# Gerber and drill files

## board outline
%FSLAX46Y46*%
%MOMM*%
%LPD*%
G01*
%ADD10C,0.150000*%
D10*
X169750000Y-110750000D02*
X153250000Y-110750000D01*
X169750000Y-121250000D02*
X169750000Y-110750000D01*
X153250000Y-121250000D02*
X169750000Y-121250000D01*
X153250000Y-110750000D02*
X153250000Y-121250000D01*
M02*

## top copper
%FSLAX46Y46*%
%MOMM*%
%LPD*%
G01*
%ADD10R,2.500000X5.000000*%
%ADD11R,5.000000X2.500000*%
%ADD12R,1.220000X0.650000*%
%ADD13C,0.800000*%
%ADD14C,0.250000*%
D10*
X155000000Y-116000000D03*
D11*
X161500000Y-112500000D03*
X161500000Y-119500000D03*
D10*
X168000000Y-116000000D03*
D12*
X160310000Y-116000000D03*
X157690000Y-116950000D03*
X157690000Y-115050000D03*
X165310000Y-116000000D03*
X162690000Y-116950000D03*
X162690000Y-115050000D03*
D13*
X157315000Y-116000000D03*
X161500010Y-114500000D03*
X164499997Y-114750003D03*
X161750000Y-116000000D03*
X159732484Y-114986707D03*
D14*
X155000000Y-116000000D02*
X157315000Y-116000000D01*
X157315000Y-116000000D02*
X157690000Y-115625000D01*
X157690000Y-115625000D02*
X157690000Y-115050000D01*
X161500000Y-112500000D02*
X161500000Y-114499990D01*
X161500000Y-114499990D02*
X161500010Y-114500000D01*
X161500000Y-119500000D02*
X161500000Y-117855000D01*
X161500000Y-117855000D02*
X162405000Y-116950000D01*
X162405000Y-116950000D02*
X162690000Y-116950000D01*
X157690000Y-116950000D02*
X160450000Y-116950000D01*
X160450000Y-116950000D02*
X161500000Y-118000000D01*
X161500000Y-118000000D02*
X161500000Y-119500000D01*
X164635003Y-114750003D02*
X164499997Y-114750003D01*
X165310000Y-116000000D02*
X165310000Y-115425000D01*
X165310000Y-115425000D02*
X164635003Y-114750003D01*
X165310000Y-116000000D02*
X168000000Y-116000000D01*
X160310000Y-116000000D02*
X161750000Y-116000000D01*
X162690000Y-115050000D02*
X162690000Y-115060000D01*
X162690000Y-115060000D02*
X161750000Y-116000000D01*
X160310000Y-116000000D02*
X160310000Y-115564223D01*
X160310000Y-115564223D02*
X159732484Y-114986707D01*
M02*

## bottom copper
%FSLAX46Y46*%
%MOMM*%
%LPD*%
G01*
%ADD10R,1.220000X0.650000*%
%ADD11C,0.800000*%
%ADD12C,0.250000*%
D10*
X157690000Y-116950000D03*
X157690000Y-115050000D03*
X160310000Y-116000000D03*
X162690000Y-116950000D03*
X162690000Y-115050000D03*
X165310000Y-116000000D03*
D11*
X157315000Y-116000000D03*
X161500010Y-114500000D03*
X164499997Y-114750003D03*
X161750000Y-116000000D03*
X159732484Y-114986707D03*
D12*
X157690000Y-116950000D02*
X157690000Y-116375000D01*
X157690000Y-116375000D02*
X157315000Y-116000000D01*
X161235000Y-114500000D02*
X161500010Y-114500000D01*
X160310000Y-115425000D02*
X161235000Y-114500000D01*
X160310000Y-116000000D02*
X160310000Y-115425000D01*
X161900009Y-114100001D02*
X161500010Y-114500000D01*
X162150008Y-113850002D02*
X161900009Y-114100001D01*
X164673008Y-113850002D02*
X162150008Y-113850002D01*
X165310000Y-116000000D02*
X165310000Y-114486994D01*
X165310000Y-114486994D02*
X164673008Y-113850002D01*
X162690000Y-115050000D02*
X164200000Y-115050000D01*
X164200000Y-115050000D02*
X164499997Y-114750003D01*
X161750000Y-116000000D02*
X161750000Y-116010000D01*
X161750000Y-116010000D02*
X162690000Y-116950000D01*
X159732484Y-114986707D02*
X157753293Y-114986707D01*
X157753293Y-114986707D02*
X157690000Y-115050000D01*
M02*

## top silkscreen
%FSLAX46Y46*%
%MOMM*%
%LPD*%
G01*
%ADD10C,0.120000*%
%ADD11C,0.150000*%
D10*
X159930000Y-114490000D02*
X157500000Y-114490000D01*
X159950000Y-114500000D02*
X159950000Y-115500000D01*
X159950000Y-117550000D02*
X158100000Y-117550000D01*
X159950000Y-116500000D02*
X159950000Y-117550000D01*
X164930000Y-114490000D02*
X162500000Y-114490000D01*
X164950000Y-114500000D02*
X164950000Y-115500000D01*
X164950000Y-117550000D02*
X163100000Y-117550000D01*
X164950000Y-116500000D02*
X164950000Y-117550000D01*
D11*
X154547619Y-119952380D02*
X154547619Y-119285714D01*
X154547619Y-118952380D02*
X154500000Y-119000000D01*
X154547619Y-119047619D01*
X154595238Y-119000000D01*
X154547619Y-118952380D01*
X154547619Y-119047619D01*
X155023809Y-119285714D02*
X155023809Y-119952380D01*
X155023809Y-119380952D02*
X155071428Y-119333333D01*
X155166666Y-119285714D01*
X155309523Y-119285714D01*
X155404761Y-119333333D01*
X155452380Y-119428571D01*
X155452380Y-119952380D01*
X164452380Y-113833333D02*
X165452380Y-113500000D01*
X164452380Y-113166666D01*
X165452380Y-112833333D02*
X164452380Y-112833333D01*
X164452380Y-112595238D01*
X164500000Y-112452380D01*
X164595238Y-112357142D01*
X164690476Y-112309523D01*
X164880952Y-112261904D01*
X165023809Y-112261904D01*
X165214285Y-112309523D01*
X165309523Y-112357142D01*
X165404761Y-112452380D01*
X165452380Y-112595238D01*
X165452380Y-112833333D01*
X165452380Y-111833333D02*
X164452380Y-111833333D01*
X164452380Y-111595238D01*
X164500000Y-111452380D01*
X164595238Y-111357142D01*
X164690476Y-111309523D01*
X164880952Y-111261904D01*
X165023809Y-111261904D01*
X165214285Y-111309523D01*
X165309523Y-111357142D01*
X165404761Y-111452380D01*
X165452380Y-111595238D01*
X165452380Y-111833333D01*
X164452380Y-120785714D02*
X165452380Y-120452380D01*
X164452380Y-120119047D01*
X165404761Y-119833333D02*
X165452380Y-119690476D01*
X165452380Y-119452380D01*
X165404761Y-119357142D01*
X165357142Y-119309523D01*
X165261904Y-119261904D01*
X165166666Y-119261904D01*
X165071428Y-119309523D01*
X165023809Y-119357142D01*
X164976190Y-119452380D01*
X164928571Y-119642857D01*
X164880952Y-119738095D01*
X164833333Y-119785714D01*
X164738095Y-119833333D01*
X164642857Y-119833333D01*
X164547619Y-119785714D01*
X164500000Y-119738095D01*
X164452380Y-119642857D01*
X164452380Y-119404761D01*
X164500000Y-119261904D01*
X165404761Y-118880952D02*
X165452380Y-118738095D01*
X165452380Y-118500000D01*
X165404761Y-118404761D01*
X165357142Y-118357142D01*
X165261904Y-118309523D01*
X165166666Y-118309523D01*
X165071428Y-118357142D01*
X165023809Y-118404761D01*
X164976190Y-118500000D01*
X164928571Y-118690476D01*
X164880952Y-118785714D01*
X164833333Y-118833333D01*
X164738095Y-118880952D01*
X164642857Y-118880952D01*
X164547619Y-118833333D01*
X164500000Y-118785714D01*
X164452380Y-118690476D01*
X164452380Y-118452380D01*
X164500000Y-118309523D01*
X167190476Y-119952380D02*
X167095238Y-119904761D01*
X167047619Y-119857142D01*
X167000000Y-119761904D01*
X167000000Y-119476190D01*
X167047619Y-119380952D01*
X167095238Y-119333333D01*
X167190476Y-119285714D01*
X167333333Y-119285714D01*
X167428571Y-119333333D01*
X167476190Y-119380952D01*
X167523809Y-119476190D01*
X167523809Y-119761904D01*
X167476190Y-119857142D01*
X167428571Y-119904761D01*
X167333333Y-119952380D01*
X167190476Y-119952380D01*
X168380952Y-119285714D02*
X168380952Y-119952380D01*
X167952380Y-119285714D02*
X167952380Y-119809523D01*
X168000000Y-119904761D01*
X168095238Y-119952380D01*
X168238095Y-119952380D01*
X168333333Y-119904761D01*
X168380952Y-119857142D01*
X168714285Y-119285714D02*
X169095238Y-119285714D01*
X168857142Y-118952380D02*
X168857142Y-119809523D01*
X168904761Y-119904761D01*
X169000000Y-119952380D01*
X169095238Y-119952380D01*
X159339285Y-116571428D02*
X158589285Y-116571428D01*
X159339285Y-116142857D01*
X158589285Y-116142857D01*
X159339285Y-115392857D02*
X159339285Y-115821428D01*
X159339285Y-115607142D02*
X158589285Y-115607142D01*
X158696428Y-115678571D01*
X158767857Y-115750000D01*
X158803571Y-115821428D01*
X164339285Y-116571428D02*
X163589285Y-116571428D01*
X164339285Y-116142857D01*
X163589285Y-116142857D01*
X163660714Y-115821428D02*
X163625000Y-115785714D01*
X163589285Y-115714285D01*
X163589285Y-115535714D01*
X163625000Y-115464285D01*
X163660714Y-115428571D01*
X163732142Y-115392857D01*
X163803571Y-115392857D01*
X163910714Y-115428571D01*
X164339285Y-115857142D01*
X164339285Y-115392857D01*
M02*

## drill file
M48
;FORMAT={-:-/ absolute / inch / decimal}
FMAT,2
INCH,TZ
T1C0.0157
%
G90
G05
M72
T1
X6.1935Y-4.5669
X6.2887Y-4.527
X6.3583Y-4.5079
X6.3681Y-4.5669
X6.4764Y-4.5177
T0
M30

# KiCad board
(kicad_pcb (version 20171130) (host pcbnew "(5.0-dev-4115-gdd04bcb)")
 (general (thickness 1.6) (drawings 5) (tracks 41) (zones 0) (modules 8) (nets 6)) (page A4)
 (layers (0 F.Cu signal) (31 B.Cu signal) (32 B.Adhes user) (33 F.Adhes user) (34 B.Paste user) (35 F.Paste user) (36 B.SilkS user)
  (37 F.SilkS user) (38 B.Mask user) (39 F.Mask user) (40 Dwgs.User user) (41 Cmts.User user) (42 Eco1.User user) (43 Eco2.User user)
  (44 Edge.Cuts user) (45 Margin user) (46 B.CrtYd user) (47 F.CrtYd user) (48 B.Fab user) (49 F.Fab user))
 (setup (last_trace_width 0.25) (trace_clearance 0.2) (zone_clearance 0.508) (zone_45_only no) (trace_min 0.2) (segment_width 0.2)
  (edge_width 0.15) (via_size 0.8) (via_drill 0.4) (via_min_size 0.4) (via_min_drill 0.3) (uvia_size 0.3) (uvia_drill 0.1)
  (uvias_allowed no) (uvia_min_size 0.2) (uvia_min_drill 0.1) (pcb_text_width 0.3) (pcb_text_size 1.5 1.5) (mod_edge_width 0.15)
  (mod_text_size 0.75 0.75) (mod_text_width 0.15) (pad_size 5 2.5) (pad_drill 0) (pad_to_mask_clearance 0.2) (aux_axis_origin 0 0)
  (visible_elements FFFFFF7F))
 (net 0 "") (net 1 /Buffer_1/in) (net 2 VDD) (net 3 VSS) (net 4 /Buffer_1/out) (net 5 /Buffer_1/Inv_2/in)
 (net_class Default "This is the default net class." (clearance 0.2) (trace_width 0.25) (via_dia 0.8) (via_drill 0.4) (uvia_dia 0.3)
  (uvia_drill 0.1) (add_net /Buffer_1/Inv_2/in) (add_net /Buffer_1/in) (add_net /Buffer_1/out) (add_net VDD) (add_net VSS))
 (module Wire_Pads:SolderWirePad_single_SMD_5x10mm (layer F.Cu) (at 155 116 90)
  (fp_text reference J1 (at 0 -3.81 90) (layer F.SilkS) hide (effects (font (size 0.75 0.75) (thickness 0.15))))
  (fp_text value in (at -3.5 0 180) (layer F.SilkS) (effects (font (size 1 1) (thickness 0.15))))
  (pad 1 smd rect (at 0 0 90) (size 5 2.5) (layers F.Cu F.Paste F.Mask) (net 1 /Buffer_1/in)))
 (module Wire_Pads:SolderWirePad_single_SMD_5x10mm (layer F.Cu) (at 161.5 112.5)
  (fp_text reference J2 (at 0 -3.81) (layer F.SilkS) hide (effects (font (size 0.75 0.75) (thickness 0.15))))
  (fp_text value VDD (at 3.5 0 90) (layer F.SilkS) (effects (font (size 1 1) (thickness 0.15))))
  (pad 1 smd rect (at 0 0) (size 5 2.5) (layers F.Cu F.Paste F.Mask) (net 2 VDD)))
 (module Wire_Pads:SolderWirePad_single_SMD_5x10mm (layer F.Cu) (at 161.5 119.5)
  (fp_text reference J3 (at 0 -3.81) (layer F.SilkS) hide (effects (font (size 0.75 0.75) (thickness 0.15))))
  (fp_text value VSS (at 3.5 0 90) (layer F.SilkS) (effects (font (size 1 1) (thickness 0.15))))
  (pad 1 smd rect (at 0 0) (size 5 2.5) (layers F.Cu F.Paste F.Mask) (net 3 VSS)))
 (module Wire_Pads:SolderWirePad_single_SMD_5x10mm (layer F.Cu) (at 168 116 90)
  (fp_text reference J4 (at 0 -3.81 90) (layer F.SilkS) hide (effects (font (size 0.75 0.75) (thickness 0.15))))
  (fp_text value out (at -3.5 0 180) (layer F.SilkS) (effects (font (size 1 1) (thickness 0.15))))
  (pad 1 smd rect (at 0 0 90) (size 5 2.5) (layers F.Cu F.Paste F.Mask) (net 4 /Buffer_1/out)))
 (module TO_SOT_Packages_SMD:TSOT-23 (layer F.Cu) (at 159 116)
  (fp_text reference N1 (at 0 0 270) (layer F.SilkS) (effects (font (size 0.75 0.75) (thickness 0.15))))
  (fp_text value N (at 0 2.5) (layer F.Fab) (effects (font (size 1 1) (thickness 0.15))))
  (fp_line (start 0.93 -1.51) (end -1.5 -1.51) (layer F.SilkS) (width 0.12))
  (fp_line (start 0.95 -1.5) (end 0.95 -0.5) (layer F.SilkS) (width 0.12))
  (fp_line (start 0.95 1.55) (end -0.9 1.55) (layer F.SilkS) (width 0.12))
  (fp_line (start 0.95 0.5) (end 0.95 1.55) (layer F.SilkS) (width 0.12))
  (pad 3 smd rect (at 1.31 0) (size 1.22 0.65) (layers F.Cu F.Paste F.Mask) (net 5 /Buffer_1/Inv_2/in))
  (pad 2 smd rect (at -1.31 0.95) (size 1.22 0.65) (layers F.Cu F.Paste F.Mask) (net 3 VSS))
  (pad 1 smd rect (at -1.31 -0.95) (size 1.22 0.65) (layers F.Cu F.Paste F.Mask) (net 1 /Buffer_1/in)))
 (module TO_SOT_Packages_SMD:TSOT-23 (layer F.Cu) (at 164 116)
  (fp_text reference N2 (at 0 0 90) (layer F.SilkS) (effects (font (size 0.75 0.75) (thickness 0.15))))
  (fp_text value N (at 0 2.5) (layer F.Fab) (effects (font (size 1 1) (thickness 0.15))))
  (fp_line (start 0.93 -1.51) (end -1.5 -1.51) (layer F.SilkS) (width 0.12))
  (fp_line (start 0.95 -1.5) (end 0.95 -0.5) (layer F.SilkS) (width 0.12))
  (fp_line (start 0.95 1.55) (end -0.9 1.55) (layer F.SilkS) (width 0.12))
  (fp_line (start 0.95 0.5) (end 0.95 1.55) (layer F.SilkS) (width 0.12))
  (pad 3 smd rect (at 1.31 0) (size 1.22 0.65) (layers F.Cu F.Paste F.Mask) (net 4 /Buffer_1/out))
  (pad 2 smd rect (at -1.31 0.95) (size 1.22 0.65) (layers F.Cu F.Paste F.Mask) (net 3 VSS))
  (pad 1 smd rect (at -1.31 -0.95) (size 1.22 0.65) (layers F.Cu F.Paste F.Mask) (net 5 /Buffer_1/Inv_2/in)))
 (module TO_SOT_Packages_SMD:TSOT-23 (layer B.Cu) (at 159 116)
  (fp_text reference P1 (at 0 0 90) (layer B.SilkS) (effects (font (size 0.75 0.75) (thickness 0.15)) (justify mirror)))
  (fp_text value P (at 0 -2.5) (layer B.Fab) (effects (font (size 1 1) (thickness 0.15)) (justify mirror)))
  (pad 1 smd rect (at -1.31 0.95) (size 1.22 0.65) (layers B.Cu B.Paste B.Mask) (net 1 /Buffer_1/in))
  (pad 2 smd rect (at -1.31 -0.95) (size 1.22 0.65) (layers B.Cu B.Paste B.Mask) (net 5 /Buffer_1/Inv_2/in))
  (pad 3 smd rect (at 1.31 0) (size 1.22 0.65) (layers B.Cu B.Paste B.Mask) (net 2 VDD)))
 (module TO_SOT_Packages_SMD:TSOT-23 (layer B.Cu) (at 164 116)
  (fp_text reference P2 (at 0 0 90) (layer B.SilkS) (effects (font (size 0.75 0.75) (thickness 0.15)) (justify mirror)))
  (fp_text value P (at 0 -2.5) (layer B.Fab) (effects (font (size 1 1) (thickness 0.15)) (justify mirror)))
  (pad 1 smd rect (at -1.31 0.95) (size 1.22 0.65) (layers B.Cu B.Paste B.Mask) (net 5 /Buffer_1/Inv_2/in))
  (pad 2 smd rect (at -1.31 -0.95) (size 1.22 0.65) (layers B.Cu B.Paste B.Mask) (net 4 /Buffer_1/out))
  (pad 3 smd rect (at 1.31 0) (size 1.22 0.65) (layers B.Cu B.Paste B.Mask) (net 2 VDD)))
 (gr_line (start 169.75 110.75) (end 153.25 110.75) (layer Edge.Cuts) (width 0.15))
 (gr_line (start 169.75 121.25) (end 169.75 110.75) (layer Edge.Cuts) (width 0.15))
 (gr_line (start 153.25 121.25) (end 169.75 121.25) (layer Edge.Cuts) (width 0.15))
 (gr_line (start 153.25 110.75) (end 153.25 121.25) (layer Edge.Cuts) (width 0.15))
 (segment (start 157.69 116.95) (end 157.69 116.375) (width 0.25) (layer B.Cu) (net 1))
 (segment (start 157.69 116.375) (end 157.315 116) (width 0.25) (layer B.Cu) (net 1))
 (via (at 157.315 116) (size 0.8) (drill 0.4) (layers F.Cu B.Cu) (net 1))
 (segment (start 155 116) (end 157.315 116) (width 0.25) (layer F.Cu) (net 1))
 (segment (start 157.315 116) (end 157.69 115.625) (width 0.25) (layer F.Cu) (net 1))
 (segment (start 157.69 115.625) (end 157.69 115.05) (width 0.25) (layer F.Cu) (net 1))
 (segment (start 161.235 114.5) (end 161.50001 114.5) (width 0.25) (layer B.Cu) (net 2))
 (segment (start 160.31 115.425) (end 161.235 114.5) (width 0.25) (layer B.Cu) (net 2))
 (segment (start 160.31 116) (end 160.31 115.425) (width 0.25) (layer B.Cu) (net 2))
 (segment (start 161.900009 114.100001) (end 161.50001 114.5) (width 0.25) (layer B.Cu) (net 2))
 (segment (start 162.150008 113.850002) (end 161.900009 114.100001) (width 0.25) (layer B.Cu) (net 2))
 (segment (start 164.673008 113.850002) (end 162.150008 113.850002) (width 0.25) (layer B.Cu) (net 2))
 (segment (start 165.31 116) (end 165.31 114.486994) (width 0.25) (layer B.Cu) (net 2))
 (segment (start 165.31 114.486994) (end 164.673008 113.850002) (width 0.25) (layer B.Cu) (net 2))
 (segment (start 161.5 112.5) (end 161.5 114.49999) (width 0.25) (layer F.Cu) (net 2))
 (segment (start 161.5 114.49999) (end 161.50001 114.5) (width 0.25) (layer F.Cu) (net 2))
 (via (at 161.50001 114.5) (size 0.8) (drill 0.4) (layers F.Cu B.Cu) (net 2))
 (segment (start 161.5 119.5) (end 161.5 117.855) (width 0.25) (layer F.Cu) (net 3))
 (segment (start 161.5 117.855) (end 162.405 116.95) (width 0.25) (layer F.Cu) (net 3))
 (segment (start 162.405 116.95) (end 162.69 116.95) (width 0.25) (layer F.Cu) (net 3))
 (segment (start 157.69 116.95) (end 160.45 116.95) (width 0.25) (layer F.Cu) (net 3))
 (segment (start 160.45 116.95) (end 161.5 118) (width 0.25) (layer F.Cu) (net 3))
 (segment (start 161.5 118) (end 161.5 119.5) (width 0.25) (layer F.Cu) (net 3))
 (segment (start 164.635003 114.750003) (end 164.499997 114.750003) (width 0.25) (layer F.Cu) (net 4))
 (segment (start 165.31 116) (end 165.31 115.425) (width 0.25) (layer F.Cu) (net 4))
 (segment (start 165.31 115.425) (end 164.635003 114.750003) (width 0.25) (layer F.Cu) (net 4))
 (segment (start 162.69 115.05) (end 164.2 115.05) (width 0.25) (layer B.Cu) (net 4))
 (via (at 164.499997 114.750003) (size 0.8) (drill 0.4) (layers F.Cu B.Cu) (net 4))
 (segment (start 164.2 115.05) (end 164.499997 114.750003) (width 0.25) (layer B.Cu) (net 4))
 (segment (start 165.31 116) (end 168 116) (width 0.25) (layer F.Cu) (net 4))
 (segment (start 160.31 116) (end 161.75 116) (width 0.25) (layer F.Cu) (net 5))
 (segment (start 161.75 116) (end 161.75 116.01) (width 0.25) (layer B.Cu) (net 5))
 (segment (start 161.75 116.01) (end 162.69 116.95) (width 0.25) (layer B.Cu) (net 5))
 (segment (start 162.69 115.05) (end 162.69 115.06) (width 0.25) (layer F.Cu) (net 5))
 (segment (start 162.69 115.06) (end 161.75 116) (width 0.25) (layer F.Cu) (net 5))
 (via (at 161.75 116) (size 0.8) (drill 0.4) (layers F.Cu B.Cu) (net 5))
 (segment (start 159.732484 114.986707) (end 157.753293 114.986707) (width 0.25) (layer B.Cu) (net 5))
 (segment (start 157.753293 114.986707) (end 157.69 115.05) (width 0.25) (layer B.Cu) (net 5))
 (segment (start 160.31 116) (end 160.31 115.564223) (width 0.25) (layer F.Cu) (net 5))
 (segment (start 160.31 115.564223) (end 159.732484 114.986707) (width 0.25) (layer F.Cu) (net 5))
 (via (at 159.732484 114.986707) (size 0.8) (drill 0.4) (layers F.Cu B.Cu) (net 5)))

